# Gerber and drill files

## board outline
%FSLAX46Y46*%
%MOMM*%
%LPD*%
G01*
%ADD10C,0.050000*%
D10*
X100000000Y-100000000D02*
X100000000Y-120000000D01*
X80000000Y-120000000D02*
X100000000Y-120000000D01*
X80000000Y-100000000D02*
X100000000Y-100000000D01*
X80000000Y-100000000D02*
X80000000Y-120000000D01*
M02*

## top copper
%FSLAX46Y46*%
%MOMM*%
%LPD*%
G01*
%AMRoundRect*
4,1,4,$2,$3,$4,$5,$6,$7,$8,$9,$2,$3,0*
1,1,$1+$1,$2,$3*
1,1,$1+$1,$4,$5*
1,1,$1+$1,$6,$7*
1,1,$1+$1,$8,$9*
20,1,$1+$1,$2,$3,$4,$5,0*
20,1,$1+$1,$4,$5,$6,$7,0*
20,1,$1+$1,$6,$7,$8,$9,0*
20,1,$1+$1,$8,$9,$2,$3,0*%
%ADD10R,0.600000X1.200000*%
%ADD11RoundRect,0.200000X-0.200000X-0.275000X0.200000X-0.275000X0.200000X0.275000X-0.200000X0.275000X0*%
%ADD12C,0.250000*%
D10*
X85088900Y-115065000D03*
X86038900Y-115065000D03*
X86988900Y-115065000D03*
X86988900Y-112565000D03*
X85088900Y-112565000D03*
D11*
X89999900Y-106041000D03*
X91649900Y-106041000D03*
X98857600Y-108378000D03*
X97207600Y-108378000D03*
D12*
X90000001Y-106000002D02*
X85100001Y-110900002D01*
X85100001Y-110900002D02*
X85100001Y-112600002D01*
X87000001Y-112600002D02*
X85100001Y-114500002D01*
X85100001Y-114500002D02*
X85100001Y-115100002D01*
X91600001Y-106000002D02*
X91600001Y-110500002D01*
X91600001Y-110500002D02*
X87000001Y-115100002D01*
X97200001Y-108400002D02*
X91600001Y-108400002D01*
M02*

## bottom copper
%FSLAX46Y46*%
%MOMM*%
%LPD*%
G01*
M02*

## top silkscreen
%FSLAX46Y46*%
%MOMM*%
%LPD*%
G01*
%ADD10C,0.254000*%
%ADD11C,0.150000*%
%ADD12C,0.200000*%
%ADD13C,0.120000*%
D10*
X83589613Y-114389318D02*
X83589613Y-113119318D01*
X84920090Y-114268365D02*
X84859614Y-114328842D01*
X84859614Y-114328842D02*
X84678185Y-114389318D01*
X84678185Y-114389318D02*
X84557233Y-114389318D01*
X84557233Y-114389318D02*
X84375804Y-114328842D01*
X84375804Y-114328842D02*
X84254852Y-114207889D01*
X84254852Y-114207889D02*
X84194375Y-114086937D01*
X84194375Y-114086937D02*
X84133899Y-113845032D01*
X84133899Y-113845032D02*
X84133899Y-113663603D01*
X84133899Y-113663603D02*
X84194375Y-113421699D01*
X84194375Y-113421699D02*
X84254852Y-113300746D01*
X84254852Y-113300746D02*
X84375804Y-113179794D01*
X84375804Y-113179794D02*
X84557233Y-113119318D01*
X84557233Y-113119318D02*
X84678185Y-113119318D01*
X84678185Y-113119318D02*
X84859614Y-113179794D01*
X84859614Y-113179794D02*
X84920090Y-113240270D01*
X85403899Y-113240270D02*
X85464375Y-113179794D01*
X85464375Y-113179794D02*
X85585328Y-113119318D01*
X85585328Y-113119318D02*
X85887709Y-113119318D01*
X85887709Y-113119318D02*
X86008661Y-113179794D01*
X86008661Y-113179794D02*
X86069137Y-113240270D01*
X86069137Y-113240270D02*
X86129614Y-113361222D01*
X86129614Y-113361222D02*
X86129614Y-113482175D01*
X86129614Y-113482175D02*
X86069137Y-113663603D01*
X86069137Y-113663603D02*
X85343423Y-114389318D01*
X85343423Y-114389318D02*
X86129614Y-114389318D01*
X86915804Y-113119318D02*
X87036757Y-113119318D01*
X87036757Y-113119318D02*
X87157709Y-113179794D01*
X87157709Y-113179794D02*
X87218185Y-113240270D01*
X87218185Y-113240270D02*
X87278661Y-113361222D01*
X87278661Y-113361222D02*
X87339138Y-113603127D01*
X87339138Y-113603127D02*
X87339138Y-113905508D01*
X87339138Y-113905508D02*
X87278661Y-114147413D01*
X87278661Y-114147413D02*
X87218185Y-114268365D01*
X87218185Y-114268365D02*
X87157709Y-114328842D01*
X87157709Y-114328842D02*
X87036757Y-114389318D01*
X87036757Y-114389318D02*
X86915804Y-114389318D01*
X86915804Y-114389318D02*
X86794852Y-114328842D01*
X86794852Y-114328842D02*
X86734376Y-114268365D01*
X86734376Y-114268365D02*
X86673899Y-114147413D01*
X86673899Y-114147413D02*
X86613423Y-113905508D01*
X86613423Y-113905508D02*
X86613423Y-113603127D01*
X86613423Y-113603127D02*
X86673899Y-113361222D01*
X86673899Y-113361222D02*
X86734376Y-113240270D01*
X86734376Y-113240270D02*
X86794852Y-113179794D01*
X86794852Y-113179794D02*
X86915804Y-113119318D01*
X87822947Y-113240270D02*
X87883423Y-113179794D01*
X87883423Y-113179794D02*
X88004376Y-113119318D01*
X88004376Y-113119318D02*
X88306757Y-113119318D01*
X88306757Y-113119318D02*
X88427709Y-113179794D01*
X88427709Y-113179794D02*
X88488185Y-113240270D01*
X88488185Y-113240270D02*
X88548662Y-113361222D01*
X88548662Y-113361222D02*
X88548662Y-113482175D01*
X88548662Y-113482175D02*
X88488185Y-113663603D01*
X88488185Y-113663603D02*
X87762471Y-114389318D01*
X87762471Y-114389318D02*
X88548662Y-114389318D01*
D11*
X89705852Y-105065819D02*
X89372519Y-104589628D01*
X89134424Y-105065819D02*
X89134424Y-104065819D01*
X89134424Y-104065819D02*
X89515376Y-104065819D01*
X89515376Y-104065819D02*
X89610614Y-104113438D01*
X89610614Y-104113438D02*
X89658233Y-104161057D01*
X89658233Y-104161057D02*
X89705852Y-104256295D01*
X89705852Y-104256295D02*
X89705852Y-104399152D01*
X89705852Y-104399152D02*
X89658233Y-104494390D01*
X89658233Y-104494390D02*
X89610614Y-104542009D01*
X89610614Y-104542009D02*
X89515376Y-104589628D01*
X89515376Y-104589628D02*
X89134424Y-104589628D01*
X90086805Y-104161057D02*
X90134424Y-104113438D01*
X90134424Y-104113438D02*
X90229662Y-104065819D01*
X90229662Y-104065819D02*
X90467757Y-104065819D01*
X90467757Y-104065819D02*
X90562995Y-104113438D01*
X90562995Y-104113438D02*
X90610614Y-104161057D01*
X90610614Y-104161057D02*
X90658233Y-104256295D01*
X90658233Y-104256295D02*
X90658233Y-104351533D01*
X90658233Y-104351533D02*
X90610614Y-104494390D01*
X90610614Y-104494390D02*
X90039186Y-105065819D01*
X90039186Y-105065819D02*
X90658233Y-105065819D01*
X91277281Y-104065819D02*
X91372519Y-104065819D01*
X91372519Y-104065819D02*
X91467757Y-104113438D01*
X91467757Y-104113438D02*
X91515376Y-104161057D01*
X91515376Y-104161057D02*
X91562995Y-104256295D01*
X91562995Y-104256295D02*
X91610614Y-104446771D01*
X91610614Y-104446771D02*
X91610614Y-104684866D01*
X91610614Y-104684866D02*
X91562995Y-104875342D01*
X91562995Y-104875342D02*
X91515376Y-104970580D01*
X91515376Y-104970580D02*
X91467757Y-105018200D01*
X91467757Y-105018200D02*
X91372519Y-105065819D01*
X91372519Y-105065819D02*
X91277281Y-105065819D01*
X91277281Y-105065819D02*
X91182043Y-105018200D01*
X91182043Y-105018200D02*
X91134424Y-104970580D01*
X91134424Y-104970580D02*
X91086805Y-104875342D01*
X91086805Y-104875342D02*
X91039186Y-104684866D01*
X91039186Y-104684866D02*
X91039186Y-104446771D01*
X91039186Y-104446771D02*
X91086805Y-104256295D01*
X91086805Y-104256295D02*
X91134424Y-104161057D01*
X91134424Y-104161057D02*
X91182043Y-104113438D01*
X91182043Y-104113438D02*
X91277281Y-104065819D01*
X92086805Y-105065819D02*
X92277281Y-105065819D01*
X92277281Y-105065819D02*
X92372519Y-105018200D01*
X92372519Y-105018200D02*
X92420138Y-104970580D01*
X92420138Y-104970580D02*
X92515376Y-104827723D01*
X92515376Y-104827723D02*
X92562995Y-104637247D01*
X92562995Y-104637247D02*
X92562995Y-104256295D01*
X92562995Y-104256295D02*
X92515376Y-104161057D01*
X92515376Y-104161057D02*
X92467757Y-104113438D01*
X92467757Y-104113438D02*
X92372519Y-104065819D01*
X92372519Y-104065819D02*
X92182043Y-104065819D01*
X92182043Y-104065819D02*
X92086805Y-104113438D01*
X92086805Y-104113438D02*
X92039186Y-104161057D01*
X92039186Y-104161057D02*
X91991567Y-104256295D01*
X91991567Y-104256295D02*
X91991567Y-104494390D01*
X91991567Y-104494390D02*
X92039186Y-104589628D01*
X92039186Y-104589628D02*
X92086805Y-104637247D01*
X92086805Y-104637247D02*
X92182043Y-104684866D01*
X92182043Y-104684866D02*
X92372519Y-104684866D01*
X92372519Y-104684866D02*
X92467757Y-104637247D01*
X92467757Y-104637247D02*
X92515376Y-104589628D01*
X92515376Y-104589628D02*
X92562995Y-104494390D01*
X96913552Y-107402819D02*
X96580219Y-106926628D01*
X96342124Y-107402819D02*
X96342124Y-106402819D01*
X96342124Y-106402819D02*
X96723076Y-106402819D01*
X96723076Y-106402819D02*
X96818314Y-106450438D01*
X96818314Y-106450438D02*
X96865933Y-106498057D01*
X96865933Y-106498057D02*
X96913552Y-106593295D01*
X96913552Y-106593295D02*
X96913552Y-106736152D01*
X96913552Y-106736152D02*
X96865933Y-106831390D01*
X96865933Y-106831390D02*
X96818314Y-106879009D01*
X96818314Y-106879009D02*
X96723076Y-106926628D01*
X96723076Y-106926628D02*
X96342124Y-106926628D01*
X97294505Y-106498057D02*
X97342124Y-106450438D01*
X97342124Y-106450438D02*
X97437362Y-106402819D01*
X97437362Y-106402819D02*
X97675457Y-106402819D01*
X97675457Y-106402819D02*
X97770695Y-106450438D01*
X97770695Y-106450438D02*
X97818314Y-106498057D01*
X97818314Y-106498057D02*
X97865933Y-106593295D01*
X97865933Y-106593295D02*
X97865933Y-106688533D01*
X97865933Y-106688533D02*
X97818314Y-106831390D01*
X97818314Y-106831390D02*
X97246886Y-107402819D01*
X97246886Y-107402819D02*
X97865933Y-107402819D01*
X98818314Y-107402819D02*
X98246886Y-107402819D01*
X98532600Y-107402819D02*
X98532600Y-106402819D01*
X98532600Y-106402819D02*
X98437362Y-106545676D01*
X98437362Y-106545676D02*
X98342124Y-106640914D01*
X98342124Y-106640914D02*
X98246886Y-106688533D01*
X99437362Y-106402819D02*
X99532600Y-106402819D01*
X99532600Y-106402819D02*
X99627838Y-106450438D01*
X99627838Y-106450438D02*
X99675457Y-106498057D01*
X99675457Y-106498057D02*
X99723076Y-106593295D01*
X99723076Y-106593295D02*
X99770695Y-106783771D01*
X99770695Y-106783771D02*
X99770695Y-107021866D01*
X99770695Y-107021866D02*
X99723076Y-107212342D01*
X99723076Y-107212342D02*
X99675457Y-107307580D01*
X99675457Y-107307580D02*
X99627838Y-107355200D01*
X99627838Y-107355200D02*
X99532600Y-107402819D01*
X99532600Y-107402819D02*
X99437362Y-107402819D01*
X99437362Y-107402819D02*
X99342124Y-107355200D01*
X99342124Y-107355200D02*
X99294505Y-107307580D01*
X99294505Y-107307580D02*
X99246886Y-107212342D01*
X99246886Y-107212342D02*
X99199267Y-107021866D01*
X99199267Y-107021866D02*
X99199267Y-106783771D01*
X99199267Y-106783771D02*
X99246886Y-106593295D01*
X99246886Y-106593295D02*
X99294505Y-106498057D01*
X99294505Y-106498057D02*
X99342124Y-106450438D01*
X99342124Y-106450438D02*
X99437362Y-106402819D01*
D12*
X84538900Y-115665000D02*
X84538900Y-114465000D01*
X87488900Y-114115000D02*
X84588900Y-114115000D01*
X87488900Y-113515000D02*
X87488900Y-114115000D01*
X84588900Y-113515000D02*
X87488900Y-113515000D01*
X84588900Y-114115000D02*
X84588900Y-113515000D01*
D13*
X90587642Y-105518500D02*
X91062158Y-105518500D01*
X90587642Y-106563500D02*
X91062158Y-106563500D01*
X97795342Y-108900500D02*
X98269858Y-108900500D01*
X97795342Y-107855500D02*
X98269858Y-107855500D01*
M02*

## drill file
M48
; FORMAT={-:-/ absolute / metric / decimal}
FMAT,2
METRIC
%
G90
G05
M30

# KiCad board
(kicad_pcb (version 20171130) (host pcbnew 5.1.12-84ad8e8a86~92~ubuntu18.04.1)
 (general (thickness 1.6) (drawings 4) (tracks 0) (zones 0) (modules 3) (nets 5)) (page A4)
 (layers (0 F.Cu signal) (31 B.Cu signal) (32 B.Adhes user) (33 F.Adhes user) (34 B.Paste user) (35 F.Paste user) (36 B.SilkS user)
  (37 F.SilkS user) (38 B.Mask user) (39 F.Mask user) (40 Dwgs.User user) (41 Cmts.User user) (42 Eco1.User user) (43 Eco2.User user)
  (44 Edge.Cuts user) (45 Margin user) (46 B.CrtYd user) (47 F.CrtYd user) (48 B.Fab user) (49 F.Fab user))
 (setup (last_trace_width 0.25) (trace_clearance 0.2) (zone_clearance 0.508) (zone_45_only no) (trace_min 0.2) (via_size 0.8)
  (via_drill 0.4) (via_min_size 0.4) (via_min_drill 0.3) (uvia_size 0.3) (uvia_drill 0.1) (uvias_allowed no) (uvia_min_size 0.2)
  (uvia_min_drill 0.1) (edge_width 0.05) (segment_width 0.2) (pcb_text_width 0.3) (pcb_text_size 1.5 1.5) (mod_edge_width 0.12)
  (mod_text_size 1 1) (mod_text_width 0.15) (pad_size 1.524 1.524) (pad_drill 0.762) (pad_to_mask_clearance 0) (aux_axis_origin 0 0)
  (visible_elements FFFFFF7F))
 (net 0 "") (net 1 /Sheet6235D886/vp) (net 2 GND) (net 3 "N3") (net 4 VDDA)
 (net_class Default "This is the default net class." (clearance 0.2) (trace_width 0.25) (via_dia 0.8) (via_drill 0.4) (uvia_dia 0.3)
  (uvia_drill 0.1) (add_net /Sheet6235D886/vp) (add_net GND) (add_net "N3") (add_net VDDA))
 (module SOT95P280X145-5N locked (layer F.Cu) (at 86.038900 113.815000 90.000000)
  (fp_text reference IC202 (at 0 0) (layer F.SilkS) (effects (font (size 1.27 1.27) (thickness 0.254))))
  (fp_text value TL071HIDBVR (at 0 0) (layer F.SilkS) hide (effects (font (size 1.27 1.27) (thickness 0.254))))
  (fp_line (start -1.85 -1.5) (end -0.65 -1.5) (layer F.SilkS) (width 0.2))
  (fp_line (start -0.3 1.45) (end -0.3 -1.45) (layer F.SilkS) (width 0.2))
  (fp_line (start 0.3 1.45) (end -0.3 1.45) (layer F.SilkS) (width 0.2))
  (fp_line (start 0.3 -1.45) (end 0.3 1.45) (layer F.SilkS) (width 0.2))
  (fp_line (start -0.3 -1.45) (end 0.3 -1.45) (layer F.SilkS) (width 0.2))
  (pad 1 smd rect (at -1.25 -0.95 180.000000) (size 0.6 1.2) (layers F.Cu F.Mask F.Paste) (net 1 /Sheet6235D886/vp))
  (pad 2 smd rect (at -1.25 0 180.000000) (size 0.6 1.2) (layers F.Cu F.Mask F.Paste) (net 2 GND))
  (pad 3 smd rect (at -1.25 0.95 180.000000) (size 0.6 1.2) (layers F.Cu F.Mask F.Paste) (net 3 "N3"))
  (pad 4 smd rect (at 1.25 0.95 180.000000) (size 0.6 1.2) (layers F.Cu F.Mask F.Paste) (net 1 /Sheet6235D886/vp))
  (pad 5 smd rect (at 1.25 -0.95 180.000000) (size 0.6 1.2) (layers F.Cu F.Mask F.Paste) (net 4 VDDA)))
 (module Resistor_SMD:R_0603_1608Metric (layer F.Cu) (at 90.824900 106.041000)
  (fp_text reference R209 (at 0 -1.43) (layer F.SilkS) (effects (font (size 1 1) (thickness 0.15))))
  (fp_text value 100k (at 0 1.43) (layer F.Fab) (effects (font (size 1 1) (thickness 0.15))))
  (fp_line (start -0.237258 -0.5225) (end 0.237258 -0.5225) (layer F.SilkS) (width 0.12))
  (fp_line (start -0.237258 0.5225) (end 0.237258 0.5225) (layer F.SilkS) (width 0.12))
  (pad 1 smd roundrect (at -0.825 0) (size 0.8 0.95) (layers F.Cu F.Mask F.Paste) (roundrect_rratio 0.25) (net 4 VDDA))
  (pad 2 smd roundrect (at 0.825 0) (size 0.8 0.95) (layers F.Cu F.Mask F.Paste) (roundrect_rratio 0.25) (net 3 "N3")))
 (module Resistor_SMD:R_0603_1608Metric (layer F.Cu) (at 98.032600 108.378000)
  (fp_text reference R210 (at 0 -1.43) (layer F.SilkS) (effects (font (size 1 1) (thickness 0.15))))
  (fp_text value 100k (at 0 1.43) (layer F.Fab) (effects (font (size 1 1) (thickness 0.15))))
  (fp_line (start -0.237258 0.5225) (end 0.237258 0.5225) (layer F.SilkS) (width 0.12))
  (fp_line (start -0.237258 -0.5225) (end 0.237258 -0.5225) (layer F.SilkS) (width 0.12))
  (pad 2 smd roundrect (at 0.825 0) (size 0.8 0.95) (layers F.Cu F.Mask F.Paste) (roundrect_rratio 0.25) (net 2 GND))
  (pad 1 smd roundrect (at -0.825 0) (size 0.8 0.95) (layers F.Cu F.Mask F.Paste) (roundrect_rratio 0.25) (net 3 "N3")))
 (gr_line (start 100 100) (end 100 120) (layer Edge.Cuts) (width 0.05))
 (gr_line (start 80 120) (end 100 120) (layer Edge.Cuts) (width 0.05))
 (gr_line (start 80 100) (end 100 100) (layer Edge.Cuts) (width 0.05))
 (gr_line (start 80 100) (end 80 120) (layer Edge.Cuts) (width 0.05))
 (segment (start 90.000001 106.000002) (end 85.100001 110.900002) (width 0.250000) (layer F.Cu) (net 4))
 (segment (start 85.100001 110.900002) (end 85.100001 112.600002) (width 0.250000) (layer F.Cu) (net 4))
 (segment (start 87.000001 112.600002) (end 85.100001 114.500002) (width 0.250000) (layer F.Cu) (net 1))
 (segment (start 85.100001 114.500002) (end 85.100001 115.100002) (width 0.250000) (layer F.Cu) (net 1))
 (segment (start 91.600001 106.000002) (end 91.600001 110.500002) (width 0.250000) (layer F.Cu) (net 3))
 (segment (start 91.600001 110.500002) (end 87.000001 115.100002) (width 0.250000) (layer F.Cu) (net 3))
 (segment (start 97.200001 108.400002) (end 91.600001 108.400002) (width 0.250000) (layer F.Cu) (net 3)))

